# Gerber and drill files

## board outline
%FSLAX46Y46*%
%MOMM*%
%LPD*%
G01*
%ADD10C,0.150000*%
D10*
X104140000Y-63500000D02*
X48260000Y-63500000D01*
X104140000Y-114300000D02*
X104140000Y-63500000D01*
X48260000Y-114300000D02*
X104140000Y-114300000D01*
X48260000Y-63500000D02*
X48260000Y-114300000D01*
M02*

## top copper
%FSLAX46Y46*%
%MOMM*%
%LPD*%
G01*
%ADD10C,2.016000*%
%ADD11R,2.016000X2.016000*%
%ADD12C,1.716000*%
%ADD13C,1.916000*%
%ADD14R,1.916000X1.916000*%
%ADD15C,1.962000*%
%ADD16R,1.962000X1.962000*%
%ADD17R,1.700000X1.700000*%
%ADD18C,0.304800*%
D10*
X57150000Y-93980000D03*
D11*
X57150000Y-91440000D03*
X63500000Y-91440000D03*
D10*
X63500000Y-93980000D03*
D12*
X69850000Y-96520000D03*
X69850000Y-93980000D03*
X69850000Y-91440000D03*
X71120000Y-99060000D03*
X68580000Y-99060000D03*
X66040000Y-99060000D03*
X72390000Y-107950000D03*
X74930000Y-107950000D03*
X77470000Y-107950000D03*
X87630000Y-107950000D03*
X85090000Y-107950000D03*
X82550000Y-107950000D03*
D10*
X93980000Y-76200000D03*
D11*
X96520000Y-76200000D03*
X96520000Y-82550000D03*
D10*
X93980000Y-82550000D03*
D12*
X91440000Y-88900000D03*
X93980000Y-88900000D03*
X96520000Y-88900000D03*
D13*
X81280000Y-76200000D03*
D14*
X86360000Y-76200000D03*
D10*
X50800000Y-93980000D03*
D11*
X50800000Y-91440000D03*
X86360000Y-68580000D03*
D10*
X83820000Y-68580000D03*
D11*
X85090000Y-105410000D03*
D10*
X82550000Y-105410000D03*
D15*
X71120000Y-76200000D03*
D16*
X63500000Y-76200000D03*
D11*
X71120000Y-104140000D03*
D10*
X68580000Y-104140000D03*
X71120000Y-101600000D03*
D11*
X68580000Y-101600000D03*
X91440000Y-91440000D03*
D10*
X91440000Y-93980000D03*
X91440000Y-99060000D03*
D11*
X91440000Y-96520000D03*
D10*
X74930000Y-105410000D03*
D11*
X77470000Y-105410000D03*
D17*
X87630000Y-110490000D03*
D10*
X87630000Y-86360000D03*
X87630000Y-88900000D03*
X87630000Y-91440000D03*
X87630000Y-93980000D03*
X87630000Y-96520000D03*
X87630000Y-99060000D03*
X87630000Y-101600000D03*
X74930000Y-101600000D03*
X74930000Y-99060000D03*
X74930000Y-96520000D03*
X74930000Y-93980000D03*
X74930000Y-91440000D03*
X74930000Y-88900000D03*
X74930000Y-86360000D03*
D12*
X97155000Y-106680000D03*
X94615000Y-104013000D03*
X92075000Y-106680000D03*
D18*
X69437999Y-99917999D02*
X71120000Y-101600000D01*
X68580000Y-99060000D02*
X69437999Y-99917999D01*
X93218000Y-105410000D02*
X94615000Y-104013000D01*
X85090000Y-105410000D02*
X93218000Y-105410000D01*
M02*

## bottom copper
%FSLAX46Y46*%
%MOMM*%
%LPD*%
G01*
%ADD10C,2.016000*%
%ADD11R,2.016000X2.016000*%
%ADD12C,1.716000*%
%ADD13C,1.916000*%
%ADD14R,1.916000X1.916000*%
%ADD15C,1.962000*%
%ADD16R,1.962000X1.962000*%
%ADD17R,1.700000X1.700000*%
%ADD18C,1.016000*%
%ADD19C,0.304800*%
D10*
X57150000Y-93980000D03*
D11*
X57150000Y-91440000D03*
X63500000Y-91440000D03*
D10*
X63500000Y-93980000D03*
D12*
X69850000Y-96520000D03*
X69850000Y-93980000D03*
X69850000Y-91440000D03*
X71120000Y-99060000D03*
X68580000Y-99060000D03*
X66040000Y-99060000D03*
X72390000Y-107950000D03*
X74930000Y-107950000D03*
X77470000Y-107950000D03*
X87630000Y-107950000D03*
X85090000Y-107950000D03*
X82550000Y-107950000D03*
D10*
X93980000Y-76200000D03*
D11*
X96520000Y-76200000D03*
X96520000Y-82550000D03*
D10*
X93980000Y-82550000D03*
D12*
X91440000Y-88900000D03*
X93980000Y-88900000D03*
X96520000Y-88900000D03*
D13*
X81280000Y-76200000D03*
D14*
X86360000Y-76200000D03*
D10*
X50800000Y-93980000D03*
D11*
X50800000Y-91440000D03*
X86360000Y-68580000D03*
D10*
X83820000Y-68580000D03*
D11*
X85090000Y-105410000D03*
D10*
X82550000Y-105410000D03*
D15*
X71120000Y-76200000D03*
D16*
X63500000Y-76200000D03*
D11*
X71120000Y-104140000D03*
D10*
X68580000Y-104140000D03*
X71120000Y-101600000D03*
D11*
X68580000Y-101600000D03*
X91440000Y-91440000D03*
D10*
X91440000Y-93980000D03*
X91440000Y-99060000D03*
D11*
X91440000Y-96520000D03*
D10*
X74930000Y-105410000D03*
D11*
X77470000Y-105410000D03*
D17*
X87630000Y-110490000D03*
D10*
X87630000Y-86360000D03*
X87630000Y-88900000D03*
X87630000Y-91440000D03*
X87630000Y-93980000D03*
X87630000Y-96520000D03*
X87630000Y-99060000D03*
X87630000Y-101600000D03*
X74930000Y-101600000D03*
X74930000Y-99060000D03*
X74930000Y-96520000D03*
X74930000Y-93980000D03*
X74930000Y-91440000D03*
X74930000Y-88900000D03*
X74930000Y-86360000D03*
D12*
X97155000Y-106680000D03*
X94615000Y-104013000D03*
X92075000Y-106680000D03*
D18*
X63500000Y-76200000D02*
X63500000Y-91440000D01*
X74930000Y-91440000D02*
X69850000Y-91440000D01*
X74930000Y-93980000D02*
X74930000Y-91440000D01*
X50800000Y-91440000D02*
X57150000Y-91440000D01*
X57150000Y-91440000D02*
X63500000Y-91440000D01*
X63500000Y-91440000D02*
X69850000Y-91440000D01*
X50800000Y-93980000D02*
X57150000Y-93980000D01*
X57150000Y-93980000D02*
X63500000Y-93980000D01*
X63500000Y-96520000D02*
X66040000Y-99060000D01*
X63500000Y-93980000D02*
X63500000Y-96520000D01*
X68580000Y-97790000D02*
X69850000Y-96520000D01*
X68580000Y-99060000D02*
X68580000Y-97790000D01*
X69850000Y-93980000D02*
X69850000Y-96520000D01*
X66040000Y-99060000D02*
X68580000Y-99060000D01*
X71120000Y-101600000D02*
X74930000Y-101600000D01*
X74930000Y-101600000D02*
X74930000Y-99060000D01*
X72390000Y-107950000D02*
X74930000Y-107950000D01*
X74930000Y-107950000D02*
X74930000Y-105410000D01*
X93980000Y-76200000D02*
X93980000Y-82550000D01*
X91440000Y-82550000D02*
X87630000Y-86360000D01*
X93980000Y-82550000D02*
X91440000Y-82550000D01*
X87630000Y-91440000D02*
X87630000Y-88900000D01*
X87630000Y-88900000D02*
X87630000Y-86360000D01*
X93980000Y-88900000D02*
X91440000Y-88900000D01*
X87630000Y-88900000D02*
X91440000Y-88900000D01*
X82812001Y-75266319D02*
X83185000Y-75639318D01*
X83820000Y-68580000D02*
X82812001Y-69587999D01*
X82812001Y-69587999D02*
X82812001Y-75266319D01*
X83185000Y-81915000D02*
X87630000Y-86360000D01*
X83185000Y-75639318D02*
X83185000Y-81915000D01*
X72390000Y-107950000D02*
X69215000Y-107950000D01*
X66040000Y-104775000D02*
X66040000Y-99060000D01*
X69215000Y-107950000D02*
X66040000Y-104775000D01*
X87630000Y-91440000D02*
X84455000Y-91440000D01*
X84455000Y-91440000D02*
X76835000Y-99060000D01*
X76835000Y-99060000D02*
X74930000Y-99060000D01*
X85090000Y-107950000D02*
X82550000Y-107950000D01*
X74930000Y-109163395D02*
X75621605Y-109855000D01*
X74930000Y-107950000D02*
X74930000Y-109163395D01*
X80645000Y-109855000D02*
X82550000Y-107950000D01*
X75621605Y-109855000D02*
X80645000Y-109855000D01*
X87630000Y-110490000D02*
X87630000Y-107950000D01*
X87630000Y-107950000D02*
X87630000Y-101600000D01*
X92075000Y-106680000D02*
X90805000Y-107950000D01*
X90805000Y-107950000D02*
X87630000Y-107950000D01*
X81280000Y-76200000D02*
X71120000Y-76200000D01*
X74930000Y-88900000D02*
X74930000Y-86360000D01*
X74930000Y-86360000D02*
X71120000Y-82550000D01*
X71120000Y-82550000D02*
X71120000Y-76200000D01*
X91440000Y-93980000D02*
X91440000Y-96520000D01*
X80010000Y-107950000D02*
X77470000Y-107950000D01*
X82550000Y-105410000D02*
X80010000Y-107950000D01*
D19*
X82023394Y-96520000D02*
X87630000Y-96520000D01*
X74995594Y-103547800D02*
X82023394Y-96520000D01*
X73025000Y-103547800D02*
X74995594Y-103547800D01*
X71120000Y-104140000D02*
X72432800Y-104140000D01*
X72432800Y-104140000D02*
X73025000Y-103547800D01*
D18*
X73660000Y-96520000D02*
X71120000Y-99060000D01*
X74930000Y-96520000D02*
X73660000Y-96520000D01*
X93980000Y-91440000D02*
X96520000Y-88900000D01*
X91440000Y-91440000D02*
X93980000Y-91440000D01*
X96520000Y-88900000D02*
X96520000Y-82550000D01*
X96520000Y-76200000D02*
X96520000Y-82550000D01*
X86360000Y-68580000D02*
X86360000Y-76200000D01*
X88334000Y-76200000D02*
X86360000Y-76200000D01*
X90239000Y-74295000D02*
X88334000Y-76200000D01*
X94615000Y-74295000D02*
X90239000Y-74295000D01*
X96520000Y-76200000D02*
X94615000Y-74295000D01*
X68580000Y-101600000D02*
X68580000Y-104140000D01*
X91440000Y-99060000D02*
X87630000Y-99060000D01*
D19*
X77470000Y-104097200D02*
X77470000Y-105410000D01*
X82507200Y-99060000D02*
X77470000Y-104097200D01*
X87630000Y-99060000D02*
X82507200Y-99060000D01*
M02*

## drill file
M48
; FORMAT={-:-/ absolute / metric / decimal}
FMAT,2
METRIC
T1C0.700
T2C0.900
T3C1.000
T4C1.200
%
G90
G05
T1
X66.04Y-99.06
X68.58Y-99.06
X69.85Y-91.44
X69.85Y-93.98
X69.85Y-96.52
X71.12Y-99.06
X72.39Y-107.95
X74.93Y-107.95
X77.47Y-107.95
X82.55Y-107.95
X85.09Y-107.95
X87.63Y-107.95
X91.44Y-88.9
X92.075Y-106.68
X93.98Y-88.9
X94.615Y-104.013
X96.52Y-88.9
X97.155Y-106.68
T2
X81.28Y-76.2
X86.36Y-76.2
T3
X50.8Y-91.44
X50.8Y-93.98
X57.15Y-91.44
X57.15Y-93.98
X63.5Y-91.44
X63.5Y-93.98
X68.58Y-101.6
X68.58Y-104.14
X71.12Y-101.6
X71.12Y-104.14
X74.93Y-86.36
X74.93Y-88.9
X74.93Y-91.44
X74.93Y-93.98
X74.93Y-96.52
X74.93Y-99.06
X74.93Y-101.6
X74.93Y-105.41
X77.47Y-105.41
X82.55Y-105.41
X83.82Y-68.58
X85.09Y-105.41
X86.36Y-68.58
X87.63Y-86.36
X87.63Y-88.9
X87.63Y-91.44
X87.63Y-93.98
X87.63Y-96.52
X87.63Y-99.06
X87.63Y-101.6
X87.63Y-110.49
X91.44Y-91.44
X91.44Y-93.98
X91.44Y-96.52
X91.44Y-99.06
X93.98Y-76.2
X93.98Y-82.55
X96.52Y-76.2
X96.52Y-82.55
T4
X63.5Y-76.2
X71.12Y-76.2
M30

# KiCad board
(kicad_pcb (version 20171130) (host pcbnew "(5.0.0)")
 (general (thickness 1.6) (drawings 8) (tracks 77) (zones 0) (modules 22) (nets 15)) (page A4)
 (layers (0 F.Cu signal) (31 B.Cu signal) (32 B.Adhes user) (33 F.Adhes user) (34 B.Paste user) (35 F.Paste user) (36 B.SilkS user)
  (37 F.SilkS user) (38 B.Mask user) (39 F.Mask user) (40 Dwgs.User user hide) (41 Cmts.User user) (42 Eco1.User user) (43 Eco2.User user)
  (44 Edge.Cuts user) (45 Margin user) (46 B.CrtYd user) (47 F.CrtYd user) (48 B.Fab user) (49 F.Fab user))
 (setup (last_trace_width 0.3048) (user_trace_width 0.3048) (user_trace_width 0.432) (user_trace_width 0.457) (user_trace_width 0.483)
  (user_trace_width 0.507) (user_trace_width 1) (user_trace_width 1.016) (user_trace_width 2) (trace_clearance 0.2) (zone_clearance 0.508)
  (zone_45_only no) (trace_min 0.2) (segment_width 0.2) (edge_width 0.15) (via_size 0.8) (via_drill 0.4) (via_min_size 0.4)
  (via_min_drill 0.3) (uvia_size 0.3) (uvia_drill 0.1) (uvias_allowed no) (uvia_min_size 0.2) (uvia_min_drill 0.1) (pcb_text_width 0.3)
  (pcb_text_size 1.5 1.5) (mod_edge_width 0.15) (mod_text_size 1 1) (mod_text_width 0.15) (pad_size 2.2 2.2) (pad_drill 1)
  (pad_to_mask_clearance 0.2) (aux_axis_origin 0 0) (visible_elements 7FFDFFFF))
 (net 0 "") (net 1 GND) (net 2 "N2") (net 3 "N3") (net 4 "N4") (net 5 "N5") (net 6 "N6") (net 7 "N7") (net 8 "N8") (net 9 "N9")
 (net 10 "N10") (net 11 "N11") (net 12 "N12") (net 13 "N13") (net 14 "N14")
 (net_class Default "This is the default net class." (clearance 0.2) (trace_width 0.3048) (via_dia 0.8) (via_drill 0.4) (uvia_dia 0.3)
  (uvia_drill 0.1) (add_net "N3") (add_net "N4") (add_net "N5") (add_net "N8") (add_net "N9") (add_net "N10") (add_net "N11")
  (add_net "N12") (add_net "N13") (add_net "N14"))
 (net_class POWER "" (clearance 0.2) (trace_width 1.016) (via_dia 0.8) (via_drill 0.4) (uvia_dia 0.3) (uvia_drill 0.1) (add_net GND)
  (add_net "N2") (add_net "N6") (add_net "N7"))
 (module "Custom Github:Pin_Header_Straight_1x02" (layer F.Cu) (at 57.15 91.44)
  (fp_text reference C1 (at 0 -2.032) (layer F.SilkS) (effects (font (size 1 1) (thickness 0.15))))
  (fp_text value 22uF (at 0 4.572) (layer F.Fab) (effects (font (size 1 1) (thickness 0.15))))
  (pad 2 thru_hole circle (at 0 2.54) (size 2.016 2.016) (drill 1) (layers *.Cu *.Mask F.SilkS) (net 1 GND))
  (pad 1 thru_hole rect (at 0 0) (size 2.016 2.016) (drill 1) (layers *.Cu *.Mask F.SilkS) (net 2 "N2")))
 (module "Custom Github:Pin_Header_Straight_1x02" (layer F.Cu) (at 63.5 91.44)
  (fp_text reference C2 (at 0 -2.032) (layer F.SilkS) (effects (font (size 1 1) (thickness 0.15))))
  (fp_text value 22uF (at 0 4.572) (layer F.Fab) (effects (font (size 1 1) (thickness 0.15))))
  (pad 1 thru_hole rect (at 0 0) (size 2.016 2.016) (drill 1) (layers *.Cu *.Mask F.SilkS) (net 2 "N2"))
  (pad 2 thru_hole circle (at 0 2.54) (size 2.016 2.016) (drill 1) (layers *.Cu *.Mask F.SilkS) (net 1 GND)))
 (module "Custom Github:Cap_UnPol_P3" (layer F.Cu) (at 69.85 91.44)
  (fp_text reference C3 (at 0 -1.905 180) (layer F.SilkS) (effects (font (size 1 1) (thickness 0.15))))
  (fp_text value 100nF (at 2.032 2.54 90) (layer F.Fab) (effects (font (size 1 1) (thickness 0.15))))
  (pad 2 thru_hole circle (at 0 5.08) (size 1.716 1.716) (drill 0.7) (layers *.Cu *.Mask F.SilkS) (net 1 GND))
  (pad 2 thru_hole circle (at 0 2.54) (size 1.716 1.716) (drill 0.7) (layers *.Cu *.Mask F.SilkS) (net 1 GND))
  (pad 1 thru_hole circle (at 0 0) (size 1.716 1.716) (drill 0.7) (layers *.Cu *.Mask F.SilkS) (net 2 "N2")))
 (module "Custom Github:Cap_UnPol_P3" (layer F.Cu) (at 71.12 99.06 270)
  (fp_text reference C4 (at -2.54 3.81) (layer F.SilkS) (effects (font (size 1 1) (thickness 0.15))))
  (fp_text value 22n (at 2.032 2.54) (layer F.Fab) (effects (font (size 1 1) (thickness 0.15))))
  (pad 1 thru_hole circle (at 0 0 270) (size 1.716 1.716) (drill 0.7) (layers *.Cu *.Mask F.SilkS) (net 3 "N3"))
  (pad 2 thru_hole circle (at 0 2.54 270) (size 1.716 1.716) (drill 0.7) (layers *.Cu *.Mask F.SilkS) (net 1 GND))
  (pad 2 thru_hole circle (at 0 5.08 270) (size 1.716 1.716) (drill 0.7) (layers *.Cu *.Mask F.SilkS) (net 1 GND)))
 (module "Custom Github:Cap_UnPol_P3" (layer F.Cu) (at 77.47 107.95 270)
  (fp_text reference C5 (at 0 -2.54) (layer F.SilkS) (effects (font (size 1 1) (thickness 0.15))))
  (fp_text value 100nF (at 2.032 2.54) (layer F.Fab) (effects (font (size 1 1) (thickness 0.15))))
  (pad 2 thru_hole circle (at 0 5.08 270) (size 1.716 1.716) (drill 0.7) (layers *.Cu *.Mask F.SilkS) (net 1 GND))
  (pad 2 thru_hole circle (at 0 2.54 270) (size 1.716 1.716) (drill 0.7) (layers *.Cu *.Mask F.SilkS) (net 1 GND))
  (pad 1 thru_hole circle (at 0 0 270) (size 1.716 1.716) (drill 0.7) (layers *.Cu *.Mask F.SilkS) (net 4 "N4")))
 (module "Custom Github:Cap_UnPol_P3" (layer F.Cu) (at 87.63 107.95 270)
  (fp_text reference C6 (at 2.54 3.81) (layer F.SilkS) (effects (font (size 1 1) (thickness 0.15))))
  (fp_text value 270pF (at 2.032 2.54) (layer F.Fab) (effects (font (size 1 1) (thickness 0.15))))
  (pad 1 thru_hole circle (at 0 0 270) (size 1.716 1.716) (drill 0.7) (layers *.Cu *.Mask F.SilkS) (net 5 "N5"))
  (pad 2 thru_hole circle (at 0 2.54 270) (size 1.716 1.716) (drill 0.7) (layers *.Cu *.Mask F.SilkS) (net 1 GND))
  (pad 2 thru_hole circle (at 0 5.08 270) (size 1.716 1.716) (drill 0.7) (layers *.Cu *.Mask F.SilkS) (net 1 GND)))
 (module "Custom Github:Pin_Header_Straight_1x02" (layer F.Cu) (at 96.52 76.2 270)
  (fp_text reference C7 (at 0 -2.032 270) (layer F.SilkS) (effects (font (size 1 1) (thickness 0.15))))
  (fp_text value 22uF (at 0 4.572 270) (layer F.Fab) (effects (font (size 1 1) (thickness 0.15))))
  (pad 2 thru_hole circle (at 0 2.54 270) (size 2.016 2.016) (drill 1) (layers *.Cu *.Mask F.SilkS) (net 1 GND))
  (pad 1 thru_hole rect (at 0 0 270) (size 2.016 2.016) (drill 1) (layers *.Cu *.Mask F.SilkS) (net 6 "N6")))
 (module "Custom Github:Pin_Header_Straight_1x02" (layer F.Cu) (at 96.52 82.55 270)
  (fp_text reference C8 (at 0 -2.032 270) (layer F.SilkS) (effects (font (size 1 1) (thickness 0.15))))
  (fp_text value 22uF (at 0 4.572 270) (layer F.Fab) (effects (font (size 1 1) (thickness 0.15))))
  (pad 1 thru_hole rect (at 0 0 270) (size 2.016 2.016) (drill 1) (layers *.Cu *.Mask F.SilkS) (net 6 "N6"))
  (pad 2 thru_hole circle (at 0 2.54 270) (size 2.016 2.016) (drill 1) (layers *.Cu *.Mask F.SilkS) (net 1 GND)))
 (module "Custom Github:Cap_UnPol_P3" (layer F.Cu) (at 96.52 88.9 270)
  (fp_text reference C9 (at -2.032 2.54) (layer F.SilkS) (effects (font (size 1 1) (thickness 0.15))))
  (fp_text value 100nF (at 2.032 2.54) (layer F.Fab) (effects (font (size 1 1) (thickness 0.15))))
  (pad 2 thru_hole circle (at 0 5.08 270) (size 1.716 1.716) (drill 0.7) (layers *.Cu *.Mask F.SilkS) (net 1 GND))
  (pad 2 thru_hole circle (at 0 2.54 270) (size 1.716 1.716) (drill 0.7) (layers *.Cu *.Mask F.SilkS) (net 1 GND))
  (pad 1 thru_hole circle (at 0 0 270) (size 1.716 1.716) (drill 0.7) (layers *.Cu *.Mask F.SilkS) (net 6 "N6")))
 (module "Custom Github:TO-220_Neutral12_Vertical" (layer F.Cu) (at 83.82 76.2 180)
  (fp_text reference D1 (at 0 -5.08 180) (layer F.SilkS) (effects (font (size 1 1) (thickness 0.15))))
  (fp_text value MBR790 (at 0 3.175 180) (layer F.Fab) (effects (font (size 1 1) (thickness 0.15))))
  (pad 2 thru_hole circle (at 2.54 0 270) (size 1.916 1.916) (drill 0.9) (layers *.Cu *.Mask F.SilkS) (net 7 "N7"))
  (pad 1 thru_hole rect (at -2.54 0 270) (size 1.916 1.916) (drill 0.9) (layers *.Cu *.Mask F.SilkS) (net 6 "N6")))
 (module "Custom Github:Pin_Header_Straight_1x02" (layer F.Cu) (at 50.8 91.44)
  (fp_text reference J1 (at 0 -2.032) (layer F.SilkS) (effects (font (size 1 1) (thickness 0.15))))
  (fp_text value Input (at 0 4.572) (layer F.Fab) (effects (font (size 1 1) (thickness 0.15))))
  (pad 2 thru_hole circle (at 0 2.54) (size 2.016 2.016) (drill 1) (layers *.Cu *.Mask F.SilkS) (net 1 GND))
  (pad 1 thru_hole rect (at 0 0) (size 2.016 2.016) (drill 1) (layers *.Cu *.Mask F.SilkS) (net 2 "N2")))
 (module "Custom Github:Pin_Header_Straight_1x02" (layer F.Cu) (at 86.36 68.58 270)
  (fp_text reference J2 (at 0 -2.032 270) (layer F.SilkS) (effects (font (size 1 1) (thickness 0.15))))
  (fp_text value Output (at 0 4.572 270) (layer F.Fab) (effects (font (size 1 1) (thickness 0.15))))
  (pad 1 thru_hole rect (at 0 0 270) (size 2.016 2.016) (drill 1) (layers *.Cu *.Mask F.SilkS) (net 6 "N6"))
  (pad 2 thru_hole circle (at 0 2.54 270) (size 2.016 2.016) (drill 1) (layers *.Cu *.Mask F.SilkS) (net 1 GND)))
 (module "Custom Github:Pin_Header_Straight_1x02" (layer F.Cu) (at 85.09 105.41 270)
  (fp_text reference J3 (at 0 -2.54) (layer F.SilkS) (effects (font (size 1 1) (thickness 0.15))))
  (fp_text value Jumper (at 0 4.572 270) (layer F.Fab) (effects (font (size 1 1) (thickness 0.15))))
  (pad 1 thru_hole rect (at 0 0 270) (size 2.016 2.016) (drill 1) (layers *.Cu *.Mask F.SilkS) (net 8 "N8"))
  (pad 2 thru_hole circle (at 0 2.54 270) (size 2.016 2.016) (drill 1) (layers *.Cu *.Mask F.SilkS) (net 4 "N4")))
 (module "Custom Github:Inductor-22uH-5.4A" (layer F.Cu) (at 67.31 76.2)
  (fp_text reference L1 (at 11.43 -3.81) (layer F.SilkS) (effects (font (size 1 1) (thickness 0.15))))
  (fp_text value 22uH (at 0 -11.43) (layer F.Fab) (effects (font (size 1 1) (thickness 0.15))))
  (pad 2 thru_hole circle (at 3.81 0) (size 1.962 1.962) (drill 1.2) (layers *.Cu *.Mask F.SilkS) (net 7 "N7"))
  (pad 1 thru_hole rect (at -3.81 0) (size 1.962 1.962) (drill 1.2) (layers *.Cu *.Mask F.SilkS) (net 2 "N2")))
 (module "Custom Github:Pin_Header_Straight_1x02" (layer F.Cu) (at 71.12 104.14 270)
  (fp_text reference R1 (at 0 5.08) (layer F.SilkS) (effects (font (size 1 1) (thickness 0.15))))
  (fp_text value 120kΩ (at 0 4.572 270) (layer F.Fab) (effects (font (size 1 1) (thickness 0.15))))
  (pad 1 thru_hole rect (at 0 0 270) (size 2.016 2.016) (drill 1) (layers *.Cu *.Mask F.SilkS) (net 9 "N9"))
  (pad 2 thru_hole circle (at 0 2.54 270) (size 2.016 2.016) (drill 1) (layers *.Cu *.Mask F.SilkS) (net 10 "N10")))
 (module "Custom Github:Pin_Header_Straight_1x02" (layer F.Cu) (at 68.58 101.6 90)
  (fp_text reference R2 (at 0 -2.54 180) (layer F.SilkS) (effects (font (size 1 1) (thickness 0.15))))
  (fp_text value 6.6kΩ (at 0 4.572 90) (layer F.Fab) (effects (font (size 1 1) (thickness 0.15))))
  (pad 2 thru_hole circle (at 0 2.54 90) (size 2.016 2.016) (drill 1) (layers *.Cu *.Mask F.SilkS) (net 1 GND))
  (pad 1 thru_hole rect (at 0 0 90) (size 2.016 2.016) (drill 1) (layers *.Cu *.Mask F.SilkS) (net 10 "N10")))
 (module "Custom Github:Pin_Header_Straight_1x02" (layer F.Cu) (at 91.44 91.44)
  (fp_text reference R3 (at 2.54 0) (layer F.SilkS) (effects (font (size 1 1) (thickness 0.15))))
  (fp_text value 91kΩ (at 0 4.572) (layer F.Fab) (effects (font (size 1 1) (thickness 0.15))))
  (pad 1 thru_hole rect (at 0 0) (size 2.016 2.016) (drill 1) (layers *.Cu *.Mask F.SilkS) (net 6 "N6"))
  (pad 2 thru_hole circle (at 0 2.54) (size 2.016 2.016) (drill 1) (layers *.Cu *.Mask F.SilkS) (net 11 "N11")))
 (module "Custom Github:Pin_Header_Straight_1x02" (layer F.Cu) (at 91.44 96.52)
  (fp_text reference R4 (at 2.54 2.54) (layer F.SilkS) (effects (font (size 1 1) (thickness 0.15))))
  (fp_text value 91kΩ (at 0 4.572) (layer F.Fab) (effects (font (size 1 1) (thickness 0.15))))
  (pad 2 thru_hole circle (at 0 2.54) (size 2.016 2.016) (drill 1) (layers *.Cu *.Mask F.SilkS) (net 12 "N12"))
  (pad 1 thru_hole rect (at 0 0) (size 2.016 2.016) (drill 1) (layers *.Cu *.Mask F.SilkS) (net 11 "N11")))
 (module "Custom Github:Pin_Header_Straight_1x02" (layer F.Cu) (at 77.47 105.41 270)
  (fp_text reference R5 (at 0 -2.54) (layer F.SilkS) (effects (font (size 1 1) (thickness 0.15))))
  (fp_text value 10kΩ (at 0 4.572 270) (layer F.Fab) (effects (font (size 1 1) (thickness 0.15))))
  (pad 2 thru_hole circle (at 0 2.54 270) (size 2.016 2.016) (drill 1) (layers *.Cu *.Mask F.SilkS) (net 1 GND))
  (pad 1 thru_hole rect (at 0 0 270) (size 2.016 2.016) (drill 1) (layers *.Cu *.Mask F.SilkS) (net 12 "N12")))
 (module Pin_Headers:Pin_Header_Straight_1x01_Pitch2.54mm (layer F.Cu) (at 87.63 110.49)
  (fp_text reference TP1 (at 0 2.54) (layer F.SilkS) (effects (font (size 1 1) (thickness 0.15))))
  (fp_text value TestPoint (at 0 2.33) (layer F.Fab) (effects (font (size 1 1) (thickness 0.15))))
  (pad 1 thru_hole rect (at 0 0) (size 1.7 1.7) (drill 1) (layers *.Cu *.Mask) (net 5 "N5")))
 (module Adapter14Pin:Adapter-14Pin (layer F.Cu) (at 74.93 86.36)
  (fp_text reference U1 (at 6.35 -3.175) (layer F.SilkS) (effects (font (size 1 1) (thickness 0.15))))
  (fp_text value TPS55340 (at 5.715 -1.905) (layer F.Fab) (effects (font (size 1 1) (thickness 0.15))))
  (pad 14 thru_hole circle (at 12.7 0) (size 2.016 2.016) (drill 1) (layers *.Cu *.Mask) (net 1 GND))
  (pad 13 thru_hole circle (at 12.7 2.54) (size 2.016 2.016) (drill 1) (layers *.Cu *.Mask) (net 1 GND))
  (pad 12 thru_hole circle (at 12.7 5.08) (size 2.016 2.016) (drill 1) (layers *.Cu *.Mask) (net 1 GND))
  (pad 11 thru_hole circle (at 12.7 7.62) (size 2.016 2.016) (drill 1) (layers *.Cu *.Mask) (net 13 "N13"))
  (pad 10 thru_hole circle (at 12.7 10.16) (size 2.016 2.016) (drill 1) (layers *.Cu *.Mask) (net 9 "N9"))
  (pad 9 thru_hole circle (at 12.7 12.7) (size 2.016 2.016) (drill 1) (layers *.Cu *.Mask) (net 12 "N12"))
  (pad 8 thru_hole circle (at 12.7 15.24) (size 2.016 2.016) (drill 1) (layers *.Cu *.Mask) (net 5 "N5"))
  (pad 7 thru_hole circle (at 0 15.24) (size 2.016 2.016) (drill 1) (layers *.Cu *.Mask) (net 1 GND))
  (pad 6 thru_hole circle (at 0 12.7) (size 2.016 2.016) (drill 1) (layers *.Cu *.Mask) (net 1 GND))
  (pad 5 thru_hole circle (at 0 10.16) (size 2.016 2.016) (drill 1) (layers *.Cu *.Mask) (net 3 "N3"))
  (pad 4 thru_hole circle (at 0 7.62) (size 2.016 2.016) (drill 1) (layers *.Cu *.Mask) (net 2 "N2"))
  (pad 3 thru_hole circle (at 0 5.08) (size 2.016 2.016) (drill 1) (layers *.Cu *.Mask) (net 2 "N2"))
  (pad 2 thru_hole circle (at 0 2.54) (size 2.016 2.016) (drill 1) (layers *.Cu *.Mask) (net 7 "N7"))
  (pad 1 thru_hole circle (at 0 0) (size 2.016 2.016) (drill 1) (layers *.Cu *.Mask) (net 7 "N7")))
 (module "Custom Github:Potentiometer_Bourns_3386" (layer F.Cu) (at 92.075 106.68 180)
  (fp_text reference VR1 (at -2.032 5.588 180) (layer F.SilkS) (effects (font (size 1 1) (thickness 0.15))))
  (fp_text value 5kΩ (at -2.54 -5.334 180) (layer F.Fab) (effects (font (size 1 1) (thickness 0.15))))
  (pad 3 thru_hole circle (at -5.08 0 180) (size 1.716 1.716) (drill 0.7) (layers *.Cu *.Mask F.SilkS) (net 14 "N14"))
  (pad 2 thru_hole circle (at -2.54 2.667 180) (size 1.716 1.716) (drill 0.7) (layers *.Cu *.Mask F.SilkS) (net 8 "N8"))
  (pad 1 thru_hole circle (at 0 0 180) (size 1.716 1.716) (drill 0.7) (layers *.Cu *.Mask F.SilkS) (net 5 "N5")))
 (gr_line (start 104.14 63.5) (end 48.26 63.5) (layer Edge.Cuts) (width 0.15))
 (gr_line (start 104.14 114.3) (end 104.14 63.5) (layer Edge.Cuts) (width 0.15))
 (gr_line (start 48.26 114.3) (end 104.14 114.3) (layer Edge.Cuts) (width 0.15))
 (gr_line (start 48.26 63.5) (end 48.26 114.3) (layer Edge.Cuts) (width 0.15))
 (segment (start 63.5 76.2) (end 63.5 91.44) (width 1.016) (layer B.Cu) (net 2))
 (segment (start 74.93 91.44) (end 69.85 91.44) (width 1.016) (layer B.Cu) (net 2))
 (segment (start 74.93 93.98) (end 74.93 91.44) (width 1.016) (layer B.Cu) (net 2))
 (segment (start 50.8 91.44) (end 57.15 91.44) (width 1.016) (layer B.Cu) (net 2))
 (segment (start 57.15 91.44) (end 63.5 91.44) (width 1.016) (layer B.Cu) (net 2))
 (segment (start 63.5 91.44) (end 69.85 91.44) (width 1.016) (layer B.Cu) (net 2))
 (segment (start 50.8 93.98) (end 57.15 93.98) (width 1.016) (layer B.Cu) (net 1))
 (segment (start 57.15 93.98) (end 63.5 93.98) (width 1.016) (layer B.Cu) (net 1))
 (segment (start 63.5 96.52) (end 66.04 99.06) (width 1.016) (layer B.Cu) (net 1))
 (segment (start 63.5 93.98) (end 63.5 96.52) (width 1.016) (layer B.Cu) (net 1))
 (segment (start 68.58 97.79) (end 69.85 96.52) (width 1.016) (layer B.Cu) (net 1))
 (segment (start 68.58 99.06) (end 68.58 97.79) (width 1.016) (layer B.Cu) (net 1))
 (segment (start 69.85 93.98) (end 69.85 96.52) (width 1.016) (layer B.Cu) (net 1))
 (segment (start 66.04 99.06) (end 68.58 99.06) (width 1.016) (layer B.Cu) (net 1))
 (segment (start 71.12 101.6) (end 74.93 101.6) (width 1.016) (layer B.Cu) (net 1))
 (segment (start 74.93 101.6) (end 74.93 99.06) (width 1.016) (layer B.Cu) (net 1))
 (segment (start 72.39 107.95) (end 74.93 107.95) (width 1.016) (layer B.Cu) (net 1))
 (segment (start 74.93 107.95) (end 74.93 105.41) (width 1.016) (layer B.Cu) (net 1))
 (segment (start 93.98 76.2) (end 93.98 82.55) (width 1.016) (layer B.Cu) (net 1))
 (segment (start 91.44 82.55) (end 87.63 86.36) (width 1.016) (layer B.Cu) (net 1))
 (segment (start 93.98 82.55) (end 91.44 82.55) (width 1.016) (layer B.Cu) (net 1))
 (segment (start 87.63 91.44) (end 87.63 88.9) (width 1.016) (layer B.Cu) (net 1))
 (segment (start 87.63 88.9) (end 87.63 86.36) (width 1.016) (layer B.Cu) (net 1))
 (segment (start 93.98 88.9) (end 91.44 88.9) (width 1.016) (layer B.Cu) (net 1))
 (segment (start 87.63 88.9) (end 91.44 88.9) (width 1.016) (layer B.Cu) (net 1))
 (segment (start 82.812001 75.266319) (end 83.185 75.639318) (width 1.016) (layer B.Cu) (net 1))
 (segment (start 83.82 68.58) (end 82.812001 69.587999) (width 1.016) (layer B.Cu) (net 1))
 (segment (start 82.812001 69.587999) (end 82.812001 75.266319) (width 1.016) (layer B.Cu) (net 1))
 (segment (start 83.185 81.915) (end 87.63 86.36) (width 1.016) (layer B.Cu) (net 1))
 (segment (start 83.185 75.639318) (end 83.185 81.915) (width 1.016) (layer B.Cu) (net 1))
 (segment (start 72.39 107.95) (end 69.215 107.95) (width 1.016) (layer B.Cu) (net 1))
 (segment (start 66.04 104.775) (end 66.04 99.06) (width 1.016) (layer B.Cu) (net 1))
 (segment (start 69.215 107.95) (end 66.04 104.775) (width 1.016) (layer B.Cu) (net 1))
 (segment (start 87.63 91.44) (end 84.455 91.44) (width 1.016) (layer B.Cu) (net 1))
 (segment (start 84.455 91.44) (end 76.835 99.06) (width 1.016) (layer B.Cu) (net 1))
 (segment (start 76.835 99.06) (end 74.93 99.06) (width 1.016) (layer B.Cu) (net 1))
 (segment (start 85.09 107.95) (end 82.55 107.95) (width 1.016) (layer B.Cu) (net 1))
 (segment (start 74.93 109.163395) (end 75.621605 109.855) (width 1.016) (layer B.Cu) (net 1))
 (segment (start 74.93 107.95) (end 74.93 109.163395) (width 1.016) (layer B.Cu) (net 1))
 (segment (start 80.645 109.855) (end 82.55 107.95) (width 1.016) (layer B.Cu) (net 1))
 (segment (start 75.621605 109.855) (end 80.645 109.855) (width 1.016) (layer B.Cu) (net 1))
 (segment (start 69.437999 99.917999) (end 71.12 101.6) (width 0.3048) (layer F.Cu) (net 1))
 (segment (start 68.58 99.06) (end 69.437999 99.917999) (width 0.3048) (layer F.Cu) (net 1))
 (segment (start 87.63 110.49) (end 87.63 107.95) (width 1.016) (layer B.Cu) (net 5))
 (segment (start 87.63 107.95) (end 87.63 101.6) (width 1.016) (layer B.Cu) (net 5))
 (segment (start 92.075 106.68) (end 90.805 107.95) (width 1.016) (layer B.Cu) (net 5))
 (segment (start 90.805 107.95) (end 87.63 107.95) (width 1.016) (layer B.Cu) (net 5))
 (segment (start 81.28 76.2) (end 71.12 76.2) (width 1.016) (layer B.Cu) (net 7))
 (segment (start 74.93 88.9) (end 74.93 86.36) (width 1.016) (layer B.Cu) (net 7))
 (segment (start 74.93 86.36) (end 71.12 82.55) (width 1.016) (layer B.Cu) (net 7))
 (segment (start 71.12 82.55) (end 71.12 76.2) (width 1.016) (layer B.Cu) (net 7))
 (segment (start 91.44 93.98) (end 91.44 96.52) (width 1.016) (layer B.Cu) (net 11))
 (segment (start 80.01 107.95) (end 77.47 107.95) (width 1.016) (layer B.Cu) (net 4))
 (segment (start 82.55 105.41) (end 80.01 107.95) (width 1.016) (layer B.Cu) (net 4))
 (segment (start 82.023394 96.52) (end 87.63 96.52) (width 0.3048) (layer B.Cu) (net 9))
 (segment (start 74.995594 103.5478) (end 82.023394 96.52) (width 0.3048) (layer B.Cu) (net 9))
 (segment (start 73.025 103.5478) (end 74.995594 103.5478) (width 0.3048) (layer B.Cu) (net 9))
 (segment (start 71.12 104.14) (end 72.4328 104.14) (width 0.3048) (layer B.Cu) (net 9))
 (segment (start 72.4328 104.14) (end 73.025 103.5478) (width 0.3048) (layer B.Cu) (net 9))
 (segment (start 73.66 96.52) (end 71.12 99.06) (width 1.016) (layer B.Cu) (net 3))
 (segment (start 74.93 96.52) (end 73.66 96.52) (width 1.016) (layer B.Cu) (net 3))
 (segment (start 93.98 91.44) (end 96.52 88.9) (width 1.016) (layer B.Cu) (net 6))
 (segment (start 91.44 91.44) (end 93.98 91.44) (width 1.016) (layer B.Cu) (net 6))
 (segment (start 96.52 88.9) (end 96.52 82.55) (width 1.016) (layer B.Cu) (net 6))
 (segment (start 96.52 76.2) (end 96.52 82.55) (width 1.016) (layer B.Cu) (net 6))
 (segment (start 86.36 68.58) (end 86.36 76.2) (width 1.016) (layer B.Cu) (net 6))
 (segment (start 88.334 76.2) (end 86.36 76.2) (width 1.016) (layer B.Cu) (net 6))
 (segment (start 90.239 74.295) (end 88.334 76.2) (width 1.016) (layer B.Cu) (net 6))
 (segment (start 94.615 74.295) (end 90.239 74.295) (width 1.016) (layer B.Cu) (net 6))
 (segment (start 96.52 76.2) (end 94.615 74.295) (width 1.016) (layer B.Cu) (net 6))
 (segment (start 93.218 105.41) (end 94.615 104.013) (width 0.3048) (layer F.Cu) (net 8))
 (segment (start 85.09 105.41) (end 93.218 105.41) (width 0.3048) (layer F.Cu) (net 8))
 (segment (start 68.58 101.6) (end 68.58 104.14) (width 1.016) (layer B.Cu) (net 10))
 (segment (start 91.44 99.06) (end 87.63 99.06) (width 1.016) (layer B.Cu) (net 12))
 (segment (start 77.47 104.0972) (end 77.47 105.41) (width 0.3048) (layer B.Cu) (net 12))
 (segment (start 82.5072 99.06) (end 77.47 104.0972) (width 0.3048) (layer B.Cu) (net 12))
 (segment (start 87.63 99.06) (end 82.5072 99.06) (width 0.3048) (layer B.Cu) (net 12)))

